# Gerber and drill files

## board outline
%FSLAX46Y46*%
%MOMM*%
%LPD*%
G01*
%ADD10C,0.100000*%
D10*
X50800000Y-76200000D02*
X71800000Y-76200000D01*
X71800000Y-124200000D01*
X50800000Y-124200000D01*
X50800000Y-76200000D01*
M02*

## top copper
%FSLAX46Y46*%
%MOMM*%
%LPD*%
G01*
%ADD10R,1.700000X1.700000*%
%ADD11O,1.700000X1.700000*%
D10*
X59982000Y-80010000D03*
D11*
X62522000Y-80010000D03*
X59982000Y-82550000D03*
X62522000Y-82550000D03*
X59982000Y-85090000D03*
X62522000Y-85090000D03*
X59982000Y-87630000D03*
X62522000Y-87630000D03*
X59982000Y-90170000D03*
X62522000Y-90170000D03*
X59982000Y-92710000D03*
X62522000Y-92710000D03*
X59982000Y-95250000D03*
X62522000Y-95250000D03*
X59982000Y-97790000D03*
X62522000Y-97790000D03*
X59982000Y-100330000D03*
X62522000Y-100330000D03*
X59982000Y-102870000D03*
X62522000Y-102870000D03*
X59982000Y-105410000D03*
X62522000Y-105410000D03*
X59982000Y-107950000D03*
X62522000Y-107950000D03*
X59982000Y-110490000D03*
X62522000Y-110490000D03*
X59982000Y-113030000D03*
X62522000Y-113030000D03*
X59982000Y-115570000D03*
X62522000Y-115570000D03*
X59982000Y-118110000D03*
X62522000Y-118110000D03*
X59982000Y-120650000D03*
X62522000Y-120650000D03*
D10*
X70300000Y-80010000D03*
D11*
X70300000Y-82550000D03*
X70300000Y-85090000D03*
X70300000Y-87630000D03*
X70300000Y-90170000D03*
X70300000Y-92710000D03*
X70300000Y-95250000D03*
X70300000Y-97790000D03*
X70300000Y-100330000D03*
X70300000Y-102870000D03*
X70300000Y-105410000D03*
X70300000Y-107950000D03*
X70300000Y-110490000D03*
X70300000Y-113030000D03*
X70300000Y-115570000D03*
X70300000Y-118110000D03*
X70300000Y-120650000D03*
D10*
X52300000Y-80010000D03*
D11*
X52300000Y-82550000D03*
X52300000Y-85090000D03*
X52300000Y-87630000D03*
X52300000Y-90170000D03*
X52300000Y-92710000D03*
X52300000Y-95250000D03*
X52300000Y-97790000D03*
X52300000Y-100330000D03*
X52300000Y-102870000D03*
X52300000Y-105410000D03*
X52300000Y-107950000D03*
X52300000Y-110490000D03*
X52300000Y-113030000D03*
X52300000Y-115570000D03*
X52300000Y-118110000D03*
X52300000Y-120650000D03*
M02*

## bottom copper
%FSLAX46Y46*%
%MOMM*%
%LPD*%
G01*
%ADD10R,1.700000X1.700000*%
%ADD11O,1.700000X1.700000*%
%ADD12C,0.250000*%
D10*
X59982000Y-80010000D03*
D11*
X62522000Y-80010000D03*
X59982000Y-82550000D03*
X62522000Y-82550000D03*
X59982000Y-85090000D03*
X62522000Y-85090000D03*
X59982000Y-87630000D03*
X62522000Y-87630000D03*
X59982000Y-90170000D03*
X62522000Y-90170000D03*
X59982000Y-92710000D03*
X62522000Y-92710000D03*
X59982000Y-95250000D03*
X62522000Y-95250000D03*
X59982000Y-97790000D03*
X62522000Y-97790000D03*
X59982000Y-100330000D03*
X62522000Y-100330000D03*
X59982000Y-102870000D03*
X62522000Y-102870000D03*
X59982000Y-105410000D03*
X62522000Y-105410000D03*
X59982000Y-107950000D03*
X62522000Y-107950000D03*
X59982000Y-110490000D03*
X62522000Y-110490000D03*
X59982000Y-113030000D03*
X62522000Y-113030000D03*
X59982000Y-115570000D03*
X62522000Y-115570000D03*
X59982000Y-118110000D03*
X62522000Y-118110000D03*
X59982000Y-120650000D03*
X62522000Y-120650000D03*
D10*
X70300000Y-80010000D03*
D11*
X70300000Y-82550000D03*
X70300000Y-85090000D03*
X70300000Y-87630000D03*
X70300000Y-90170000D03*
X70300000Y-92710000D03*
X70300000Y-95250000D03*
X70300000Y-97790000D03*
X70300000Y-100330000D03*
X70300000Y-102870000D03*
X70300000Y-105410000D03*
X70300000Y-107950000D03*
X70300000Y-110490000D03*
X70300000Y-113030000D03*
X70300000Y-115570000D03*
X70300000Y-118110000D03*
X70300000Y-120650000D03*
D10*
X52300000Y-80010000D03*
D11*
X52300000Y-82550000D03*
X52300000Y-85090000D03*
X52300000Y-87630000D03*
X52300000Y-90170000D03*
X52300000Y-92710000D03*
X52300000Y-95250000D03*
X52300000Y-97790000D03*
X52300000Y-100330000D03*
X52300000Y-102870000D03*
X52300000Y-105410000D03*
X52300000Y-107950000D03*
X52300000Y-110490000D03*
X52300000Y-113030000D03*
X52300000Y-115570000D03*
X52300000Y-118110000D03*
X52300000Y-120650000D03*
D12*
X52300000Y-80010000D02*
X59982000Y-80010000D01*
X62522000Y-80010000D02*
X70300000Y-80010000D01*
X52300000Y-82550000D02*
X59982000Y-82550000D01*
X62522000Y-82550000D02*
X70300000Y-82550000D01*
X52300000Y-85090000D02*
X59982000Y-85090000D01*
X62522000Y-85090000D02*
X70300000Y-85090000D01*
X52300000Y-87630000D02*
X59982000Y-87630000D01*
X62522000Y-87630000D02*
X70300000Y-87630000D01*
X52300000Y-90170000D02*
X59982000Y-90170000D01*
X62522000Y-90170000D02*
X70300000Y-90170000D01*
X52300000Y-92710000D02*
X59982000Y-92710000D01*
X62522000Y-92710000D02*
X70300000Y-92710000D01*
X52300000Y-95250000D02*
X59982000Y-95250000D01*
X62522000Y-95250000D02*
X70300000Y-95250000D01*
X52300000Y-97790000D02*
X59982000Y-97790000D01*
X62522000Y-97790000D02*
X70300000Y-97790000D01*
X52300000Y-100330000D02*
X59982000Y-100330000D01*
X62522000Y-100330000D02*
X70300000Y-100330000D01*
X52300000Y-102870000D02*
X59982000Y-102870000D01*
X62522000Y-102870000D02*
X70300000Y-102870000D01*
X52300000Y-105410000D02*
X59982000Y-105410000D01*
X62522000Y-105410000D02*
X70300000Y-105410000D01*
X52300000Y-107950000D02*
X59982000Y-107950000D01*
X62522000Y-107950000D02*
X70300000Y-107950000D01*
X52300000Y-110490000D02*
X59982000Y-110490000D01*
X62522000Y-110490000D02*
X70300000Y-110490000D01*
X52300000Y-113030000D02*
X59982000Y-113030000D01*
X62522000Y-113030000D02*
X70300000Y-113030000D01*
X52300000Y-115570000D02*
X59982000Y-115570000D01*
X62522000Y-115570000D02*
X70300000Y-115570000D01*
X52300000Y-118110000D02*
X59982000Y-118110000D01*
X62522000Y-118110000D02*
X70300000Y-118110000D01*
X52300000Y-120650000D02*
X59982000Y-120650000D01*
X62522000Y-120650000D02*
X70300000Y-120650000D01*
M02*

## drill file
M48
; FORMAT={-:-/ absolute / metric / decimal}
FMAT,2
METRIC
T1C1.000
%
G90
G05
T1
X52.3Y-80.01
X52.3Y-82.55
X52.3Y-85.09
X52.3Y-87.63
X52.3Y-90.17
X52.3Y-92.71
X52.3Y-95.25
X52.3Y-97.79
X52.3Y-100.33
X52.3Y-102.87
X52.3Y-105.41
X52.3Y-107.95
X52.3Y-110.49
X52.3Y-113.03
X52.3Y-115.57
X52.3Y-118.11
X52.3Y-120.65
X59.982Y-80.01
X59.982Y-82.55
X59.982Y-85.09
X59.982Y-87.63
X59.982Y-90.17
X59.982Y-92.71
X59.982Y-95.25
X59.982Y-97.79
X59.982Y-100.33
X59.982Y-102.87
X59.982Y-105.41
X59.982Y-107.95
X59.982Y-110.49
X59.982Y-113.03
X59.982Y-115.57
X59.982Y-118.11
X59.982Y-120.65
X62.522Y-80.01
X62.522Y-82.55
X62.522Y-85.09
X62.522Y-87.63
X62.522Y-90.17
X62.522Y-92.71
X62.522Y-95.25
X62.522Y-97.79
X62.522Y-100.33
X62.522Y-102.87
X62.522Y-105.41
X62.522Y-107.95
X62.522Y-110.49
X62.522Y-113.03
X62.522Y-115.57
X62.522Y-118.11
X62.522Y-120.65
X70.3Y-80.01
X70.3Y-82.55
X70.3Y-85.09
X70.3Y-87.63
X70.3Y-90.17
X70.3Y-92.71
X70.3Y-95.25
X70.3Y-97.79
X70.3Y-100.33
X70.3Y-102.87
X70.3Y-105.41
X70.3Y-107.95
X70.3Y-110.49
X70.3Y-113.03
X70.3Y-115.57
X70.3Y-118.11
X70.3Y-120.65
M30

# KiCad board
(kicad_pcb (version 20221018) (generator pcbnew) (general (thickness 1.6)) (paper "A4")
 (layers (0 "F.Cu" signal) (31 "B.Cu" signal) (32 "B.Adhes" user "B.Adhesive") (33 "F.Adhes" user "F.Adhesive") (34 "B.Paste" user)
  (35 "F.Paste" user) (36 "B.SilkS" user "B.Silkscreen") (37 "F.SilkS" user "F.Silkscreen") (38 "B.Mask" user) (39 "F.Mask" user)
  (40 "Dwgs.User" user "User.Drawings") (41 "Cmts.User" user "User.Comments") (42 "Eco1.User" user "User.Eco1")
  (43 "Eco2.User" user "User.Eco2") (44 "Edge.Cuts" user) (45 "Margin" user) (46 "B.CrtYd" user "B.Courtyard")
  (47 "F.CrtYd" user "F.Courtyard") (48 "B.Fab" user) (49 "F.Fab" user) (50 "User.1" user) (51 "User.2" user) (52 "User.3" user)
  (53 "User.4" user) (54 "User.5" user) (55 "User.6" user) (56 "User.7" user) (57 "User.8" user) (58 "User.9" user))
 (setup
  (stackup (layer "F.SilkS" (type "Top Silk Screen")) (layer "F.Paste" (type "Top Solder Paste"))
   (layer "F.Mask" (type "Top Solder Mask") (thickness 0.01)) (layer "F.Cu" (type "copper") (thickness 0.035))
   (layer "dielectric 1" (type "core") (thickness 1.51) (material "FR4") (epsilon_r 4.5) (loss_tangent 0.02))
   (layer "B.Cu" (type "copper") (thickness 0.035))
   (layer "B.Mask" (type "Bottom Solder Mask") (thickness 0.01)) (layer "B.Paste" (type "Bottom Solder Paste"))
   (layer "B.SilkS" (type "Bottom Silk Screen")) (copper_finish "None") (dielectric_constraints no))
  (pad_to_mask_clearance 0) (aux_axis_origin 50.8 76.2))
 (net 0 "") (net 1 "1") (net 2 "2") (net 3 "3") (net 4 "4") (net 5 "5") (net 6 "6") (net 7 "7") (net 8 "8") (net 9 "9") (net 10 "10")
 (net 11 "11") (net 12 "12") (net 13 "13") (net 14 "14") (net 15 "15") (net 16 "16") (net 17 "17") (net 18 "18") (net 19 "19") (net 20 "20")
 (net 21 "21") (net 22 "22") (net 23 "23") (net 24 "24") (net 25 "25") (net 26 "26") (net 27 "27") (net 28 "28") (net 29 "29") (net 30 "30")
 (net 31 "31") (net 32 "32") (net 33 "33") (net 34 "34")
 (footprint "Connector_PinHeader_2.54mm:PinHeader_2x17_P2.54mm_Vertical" (layer "F.Cu") (at 59.982 80.01)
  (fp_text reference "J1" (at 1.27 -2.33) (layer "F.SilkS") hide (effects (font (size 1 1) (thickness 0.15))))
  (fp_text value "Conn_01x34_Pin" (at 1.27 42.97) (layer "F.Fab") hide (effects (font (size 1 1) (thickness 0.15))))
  (pad "1" thru_hole rect (at 0 0) (size 1.7 1.7) (drill 1) (layers "*.Cu" "*.Mask") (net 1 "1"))
  (pad "2" thru_hole oval (at 2.54 0) (size 1.7 1.7) (drill 1) (layers "*.Cu" "*.Mask") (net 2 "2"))
  (pad "3" thru_hole oval (at 0 2.54) (size 1.7 1.7) (drill 1) (layers "*.Cu" "*.Mask") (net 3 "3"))
  (pad "4" thru_hole oval (at 2.54 2.54) (size 1.7 1.7) (drill 1) (layers "*.Cu" "*.Mask") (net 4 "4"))
  (pad "5" thru_hole oval (at 0 5.08) (size 1.7 1.7) (drill 1) (layers "*.Cu" "*.Mask") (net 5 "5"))
  (pad "6" thru_hole oval (at 2.54 5.08) (size 1.7 1.7) (drill 1) (layers "*.Cu" "*.Mask") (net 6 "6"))
  (pad "7" thru_hole oval (at 0 7.62) (size 1.7 1.7) (drill 1) (layers "*.Cu" "*.Mask") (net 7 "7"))
  (pad "8" thru_hole oval (at 2.54 7.62) (size 1.7 1.7) (drill 1) (layers "*.Cu" "*.Mask") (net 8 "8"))
  (pad "9" thru_hole oval (at 0 10.16) (size 1.7 1.7) (drill 1) (layers "*.Cu" "*.Mask") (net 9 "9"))
  (pad "10" thru_hole oval (at 2.54 10.16) (size 1.7 1.7) (drill 1) (layers "*.Cu" "*.Mask") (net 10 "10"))
  (pad "11" thru_hole oval (at 0 12.7) (size 1.7 1.7) (drill 1) (layers "*.Cu" "*.Mask") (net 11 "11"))
  (pad "12" thru_hole oval (at 2.54 12.7) (size 1.7 1.7) (drill 1) (layers "*.Cu" "*.Mask") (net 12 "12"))
  (pad "13" thru_hole oval (at 0 15.24) (size 1.7 1.7) (drill 1) (layers "*.Cu" "*.Mask") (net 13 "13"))
  (pad "14" thru_hole oval (at 2.54 15.24) (size 1.7 1.7) (drill 1) (layers "*.Cu" "*.Mask") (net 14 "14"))
  (pad "15" thru_hole oval (at 0 17.78) (size 1.7 1.7) (drill 1) (layers "*.Cu" "*.Mask") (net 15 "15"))
  (pad "16" thru_hole oval (at 2.54 17.78) (size 1.7 1.7) (drill 1) (layers "*.Cu" "*.Mask") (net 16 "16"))
  (pad "17" thru_hole oval (at 0 20.32) (size 1.7 1.7) (drill 1) (layers "*.Cu" "*.Mask") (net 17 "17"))
  (pad "18" thru_hole oval (at 2.54 20.32) (size 1.7 1.7) (drill 1) (layers "*.Cu" "*.Mask") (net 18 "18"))
  (pad "19" thru_hole oval (at 0 22.86) (size 1.7 1.7) (drill 1) (layers "*.Cu" "*.Mask") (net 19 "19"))
  (pad "20" thru_hole oval (at 2.54 22.86) (size 1.7 1.7) (drill 1) (layers "*.Cu" "*.Mask") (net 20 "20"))
  (pad "21" thru_hole oval (at 0 25.4) (size 1.7 1.7) (drill 1) (layers "*.Cu" "*.Mask") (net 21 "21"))
  (pad "22" thru_hole oval (at 2.54 25.4) (size 1.7 1.7) (drill 1) (layers "*.Cu" "*.Mask") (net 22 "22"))
  (pad "23" thru_hole oval (at 0 27.94) (size 1.7 1.7) (drill 1) (layers "*.Cu" "*.Mask") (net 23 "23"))
  (pad "24" thru_hole oval (at 2.54 27.94) (size 1.7 1.7) (drill 1) (layers "*.Cu" "*.Mask") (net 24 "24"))
  (pad "25" thru_hole oval (at 0 30.48) (size 1.7 1.7) (drill 1) (layers "*.Cu" "*.Mask") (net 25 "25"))
  (pad "26" thru_hole oval (at 2.54 30.48) (size 1.7 1.7) (drill 1) (layers "*.Cu" "*.Mask") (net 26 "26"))
  (pad "27" thru_hole oval (at 0 33.02) (size 1.7 1.7) (drill 1) (layers "*.Cu" "*.Mask") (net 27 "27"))
  (pad "28" thru_hole oval (at 2.54 33.02) (size 1.7 1.7) (drill 1) (layers "*.Cu" "*.Mask") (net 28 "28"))
  (pad "29" thru_hole oval (at 0 35.56) (size 1.7 1.7) (drill 1) (layers "*.Cu" "*.Mask") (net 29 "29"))
  (pad "30" thru_hole oval (at 2.54 35.56) (size 1.7 1.7) (drill 1) (layers "*.Cu" "*.Mask") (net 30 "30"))
  (pad "31" thru_hole oval (at 0 38.1) (size 1.7 1.7) (drill 1) (layers "*.Cu" "*.Mask") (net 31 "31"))
  (pad "32" thru_hole oval (at 2.54 38.1) (size 1.7 1.7) (drill 1) (layers "*.Cu" "*.Mask") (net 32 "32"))
  (pad "33" thru_hole oval (at 0 40.64) (size 1.7 1.7) (drill 1) (layers "*.Cu" "*.Mask") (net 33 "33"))
  (pad "34" thru_hole oval (at 2.54 40.64) (size 1.7 1.7) (drill 1) (layers "*.Cu" "*.Mask") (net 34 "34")))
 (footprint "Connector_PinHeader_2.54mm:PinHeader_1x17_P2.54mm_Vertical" (layer "B.Cu") (at 70.3 80.01 180)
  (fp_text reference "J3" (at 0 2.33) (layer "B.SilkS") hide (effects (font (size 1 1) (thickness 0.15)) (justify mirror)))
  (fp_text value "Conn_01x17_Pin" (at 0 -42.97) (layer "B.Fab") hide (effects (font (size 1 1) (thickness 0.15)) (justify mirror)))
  (pad "1" thru_hole rect (at 0 0 180) (size 1.7 1.7) (drill 1) (layers "*.Cu" "*.Mask") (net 2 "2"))
  (pad "2" thru_hole oval (at 0 -2.54 180) (size 1.7 1.7) (drill 1) (layers "*.Cu" "*.Mask") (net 4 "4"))
  (pad "3" thru_hole oval (at 0 -5.08 180) (size 1.7 1.7) (drill 1) (layers "*.Cu" "*.Mask") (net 6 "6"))
  (pad "4" thru_hole oval (at 0 -7.62 180) (size 1.7 1.7) (drill 1) (layers "*.Cu" "*.Mask") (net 8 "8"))
  (pad "5" thru_hole oval (at 0 -10.16 180) (size 1.7 1.7) (drill 1) (layers "*.Cu" "*.Mask") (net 10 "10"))
  (pad "6" thru_hole oval (at 0 -12.7 180) (size 1.7 1.7) (drill 1) (layers "*.Cu" "*.Mask") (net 12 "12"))
  (pad "7" thru_hole oval (at 0 -15.24 180) (size 1.7 1.7) (drill 1) (layers "*.Cu" "*.Mask") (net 14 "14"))
  (pad "8" thru_hole oval (at 0 -17.78 180) (size 1.7 1.7) (drill 1) (layers "*.Cu" "*.Mask") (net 16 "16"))
  (pad "9" thru_hole oval (at 0 -20.32 180) (size 1.7 1.7) (drill 1) (layers "*.Cu" "*.Mask") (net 18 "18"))
  (pad "10" thru_hole oval (at 0 -22.86 180) (size 1.7 1.7) (drill 1) (layers "*.Cu" "*.Mask") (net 20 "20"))
  (pad "11" thru_hole oval (at 0 -25.4 180) (size 1.7 1.7) (drill 1) (layers "*.Cu" "*.Mask") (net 22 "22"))
  (pad "12" thru_hole oval (at 0 -27.94 180) (size 1.7 1.7) (drill 1) (layers "*.Cu" "*.Mask") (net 24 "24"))
  (pad "13" thru_hole oval (at 0 -30.48 180) (size 1.7 1.7) (drill 1) (layers "*.Cu" "*.Mask") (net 26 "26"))
  (pad "14" thru_hole oval (at 0 -33.02 180) (size 1.7 1.7) (drill 1) (layers "*.Cu" "*.Mask") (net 28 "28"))
  (pad "15" thru_hole oval (at 0 -35.56 180) (size 1.7 1.7) (drill 1) (layers "*.Cu" "*.Mask") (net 30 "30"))
  (pad "16" thru_hole oval (at 0 -38.1 180) (size 1.7 1.7) (drill 1) (layers "*.Cu" "*.Mask") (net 32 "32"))
  (pad "17" thru_hole oval (at 0 -40.64 180) (size 1.7 1.7) (drill 1) (layers "*.Cu" "*.Mask") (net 34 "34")))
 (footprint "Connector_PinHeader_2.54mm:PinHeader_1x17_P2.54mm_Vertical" (layer "B.Cu") (at 52.3 80.01 180)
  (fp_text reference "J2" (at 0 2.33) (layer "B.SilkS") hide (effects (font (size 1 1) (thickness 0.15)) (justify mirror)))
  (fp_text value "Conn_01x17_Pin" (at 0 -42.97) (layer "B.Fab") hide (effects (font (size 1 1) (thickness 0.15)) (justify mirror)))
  (pad "1" thru_hole rect (at 0 0 180) (size 1.7 1.7) (drill 1) (layers "*.Cu" "*.Mask") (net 1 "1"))
  (pad "2" thru_hole oval (at 0 -2.54 180) (size 1.7 1.7) (drill 1) (layers "*.Cu" "*.Mask") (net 3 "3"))
  (pad "3" thru_hole oval (at 0 -5.08 180) (size 1.7 1.7) (drill 1) (layers "*.Cu" "*.Mask") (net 5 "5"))
  (pad "4" thru_hole oval (at 0 -7.62 180) (size 1.7 1.7) (drill 1) (layers "*.Cu" "*.Mask") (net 7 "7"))
  (pad "5" thru_hole oval (at 0 -10.16 180) (size 1.7 1.7) (drill 1) (layers "*.Cu" "*.Mask") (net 9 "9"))
  (pad "6" thru_hole oval (at 0 -12.7 180) (size 1.7 1.7) (drill 1) (layers "*.Cu" "*.Mask") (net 11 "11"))
  (pad "7" thru_hole oval (at 0 -15.24 180) (size 1.7 1.7) (drill 1) (layers "*.Cu" "*.Mask") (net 13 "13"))
  (pad "8" thru_hole oval (at 0 -17.78 180) (size 1.7 1.7) (drill 1) (layers "*.Cu" "*.Mask") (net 15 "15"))
  (pad "9" thru_hole oval (at 0 -20.32 180) (size 1.7 1.7) (drill 1) (layers "*.Cu" "*.Mask") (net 17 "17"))
  (pad "10" thru_hole oval (at 0 -22.86 180) (size 1.7 1.7) (drill 1) (layers "*.Cu" "*.Mask") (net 19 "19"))
  (pad "11" thru_hole oval (at 0 -25.4 180) (size 1.7 1.7) (drill 1) (layers "*.Cu" "*.Mask") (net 21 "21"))
  (pad "12" thru_hole oval (at 0 -27.94 180) (size 1.7 1.7) (drill 1) (layers "*.Cu" "*.Mask") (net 23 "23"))
  (pad "13" thru_hole oval (at 0 -30.48 180) (size 1.7 1.7) (drill 1) (layers "*.Cu" "*.Mask") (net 25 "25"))
  (pad "14" thru_hole oval (at 0 -33.02 180) (size 1.7 1.7) (drill 1) (layers "*.Cu" "*.Mask") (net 27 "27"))
  (pad "15" thru_hole oval (at 0 -35.56 180) (size 1.7 1.7) (drill 1) (layers "*.Cu" "*.Mask") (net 29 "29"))
  (pad "16" thru_hole oval (at 0 -38.1 180) (size 1.7 1.7) (drill 1) (layers "*.Cu" "*.Mask") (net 31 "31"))
  (pad "17" thru_hole oval (at 0 -40.64 180) (size 1.7 1.7) (drill 1) (layers "*.Cu" "*.Mask") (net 33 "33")))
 (gr_rect (start 50.8 76.2) (end 71.8 124.2) (stroke (width 0.1) (type default)) (fill none) (layer "Edge.Cuts"))
 (segment (start 52.3 80.01) (end 59.982 80.01) (width 0.25) (layer "B.Cu") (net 1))
 (segment (start 62.522 80.01) (end 70.3 80.01) (width 0.25) (layer "B.Cu") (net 2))
 (segment (start 52.3 82.55) (end 59.982 82.55) (width 0.25) (layer "B.Cu") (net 3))
 (segment (start 62.522 82.55) (end 70.3 82.55) (width 0.25) (layer "B.Cu") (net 4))
 (segment (start 52.3 85.09) (end 59.982 85.09) (width 0.25) (layer "B.Cu") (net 5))
 (segment (start 62.522 85.09) (end 70.3 85.09) (width 0.25) (layer "B.Cu") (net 6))
 (segment (start 52.3 87.63) (end 59.982 87.63) (width 0.25) (layer "B.Cu") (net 7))
 (segment (start 62.522 87.63) (end 70.3 87.63) (width 0.25) (layer "B.Cu") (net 8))
 (segment (start 52.3 90.17) (end 59.982 90.17) (width 0.25) (layer "B.Cu") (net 9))
 (segment (start 62.522 90.17) (end 70.3 90.17) (width 0.25) (layer "B.Cu") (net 10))
 (segment (start 52.3 92.71) (end 59.982 92.71) (width 0.25) (layer "B.Cu") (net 11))
 (segment (start 62.522 92.71) (end 70.3 92.71) (width 0.25) (layer "B.Cu") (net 12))
 (segment (start 52.3 95.25) (end 59.982 95.25) (width 0.25) (layer "B.Cu") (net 13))
 (segment (start 62.522 95.25) (end 70.3 95.25) (width 0.25) (layer "B.Cu") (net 14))
 (segment (start 52.3 97.79) (end 59.982 97.79) (width 0.25) (layer "B.Cu") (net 15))
 (segment (start 62.522 97.79) (end 70.3 97.79) (width 0.25) (layer "B.Cu") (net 16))
 (segment (start 52.3 100.33) (end 59.982 100.33) (width 0.25) (layer "B.Cu") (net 17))
 (segment (start 62.522 100.33) (end 70.3 100.33) (width 0.25) (layer "B.Cu") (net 18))
 (segment (start 52.3 102.87) (end 59.982 102.87) (width 0.25) (layer "B.Cu") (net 19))
 (segment (start 62.522 102.87) (end 70.3 102.87) (width 0.25) (layer "B.Cu") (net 20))
 (segment (start 52.3 105.41) (end 59.982 105.41) (width 0.25) (layer "B.Cu") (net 21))
 (segment (start 62.522 105.41) (end 70.3 105.41) (width 0.25) (layer "B.Cu") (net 22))
 (segment (start 52.3 107.95) (end 59.982 107.95) (width 0.25) (layer "B.Cu") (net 23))
 (segment (start 62.522 107.95) (end 70.3 107.95) (width 0.25) (layer "B.Cu") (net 24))
 (segment (start 52.3 110.49) (end 59.982 110.49) (width 0.25) (layer "B.Cu") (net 25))
 (segment (start 62.522 110.49) (end 70.3 110.49) (width 0.25) (layer "B.Cu") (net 26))
 (segment (start 52.3 113.03) (end 59.982 113.03) (width 0.25) (layer "B.Cu") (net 27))
 (segment (start 62.522 113.03) (end 70.3 113.03) (width 0.25) (layer "B.Cu") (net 28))
 (segment (start 52.3 115.57) (end 59.982 115.57) (width 0.25) (layer "B.Cu") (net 29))
 (segment (start 62.522 115.57) (end 70.3 115.57) (width 0.25) (layer "B.Cu") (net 30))
 (segment (start 52.3 118.11) (end 59.982 118.11) (width 0.25) (layer "B.Cu") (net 31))
 (segment (start 62.522 118.11) (end 70.3 118.11) (width 0.25) (layer "B.Cu") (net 32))
 (segment (start 52.3 120.65) (end 59.982 120.65) (width 0.25) (layer "B.Cu") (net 33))
 (segment (start 62.522 120.65) (end 70.3 120.65) (width 0.25) (layer "B.Cu") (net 34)))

